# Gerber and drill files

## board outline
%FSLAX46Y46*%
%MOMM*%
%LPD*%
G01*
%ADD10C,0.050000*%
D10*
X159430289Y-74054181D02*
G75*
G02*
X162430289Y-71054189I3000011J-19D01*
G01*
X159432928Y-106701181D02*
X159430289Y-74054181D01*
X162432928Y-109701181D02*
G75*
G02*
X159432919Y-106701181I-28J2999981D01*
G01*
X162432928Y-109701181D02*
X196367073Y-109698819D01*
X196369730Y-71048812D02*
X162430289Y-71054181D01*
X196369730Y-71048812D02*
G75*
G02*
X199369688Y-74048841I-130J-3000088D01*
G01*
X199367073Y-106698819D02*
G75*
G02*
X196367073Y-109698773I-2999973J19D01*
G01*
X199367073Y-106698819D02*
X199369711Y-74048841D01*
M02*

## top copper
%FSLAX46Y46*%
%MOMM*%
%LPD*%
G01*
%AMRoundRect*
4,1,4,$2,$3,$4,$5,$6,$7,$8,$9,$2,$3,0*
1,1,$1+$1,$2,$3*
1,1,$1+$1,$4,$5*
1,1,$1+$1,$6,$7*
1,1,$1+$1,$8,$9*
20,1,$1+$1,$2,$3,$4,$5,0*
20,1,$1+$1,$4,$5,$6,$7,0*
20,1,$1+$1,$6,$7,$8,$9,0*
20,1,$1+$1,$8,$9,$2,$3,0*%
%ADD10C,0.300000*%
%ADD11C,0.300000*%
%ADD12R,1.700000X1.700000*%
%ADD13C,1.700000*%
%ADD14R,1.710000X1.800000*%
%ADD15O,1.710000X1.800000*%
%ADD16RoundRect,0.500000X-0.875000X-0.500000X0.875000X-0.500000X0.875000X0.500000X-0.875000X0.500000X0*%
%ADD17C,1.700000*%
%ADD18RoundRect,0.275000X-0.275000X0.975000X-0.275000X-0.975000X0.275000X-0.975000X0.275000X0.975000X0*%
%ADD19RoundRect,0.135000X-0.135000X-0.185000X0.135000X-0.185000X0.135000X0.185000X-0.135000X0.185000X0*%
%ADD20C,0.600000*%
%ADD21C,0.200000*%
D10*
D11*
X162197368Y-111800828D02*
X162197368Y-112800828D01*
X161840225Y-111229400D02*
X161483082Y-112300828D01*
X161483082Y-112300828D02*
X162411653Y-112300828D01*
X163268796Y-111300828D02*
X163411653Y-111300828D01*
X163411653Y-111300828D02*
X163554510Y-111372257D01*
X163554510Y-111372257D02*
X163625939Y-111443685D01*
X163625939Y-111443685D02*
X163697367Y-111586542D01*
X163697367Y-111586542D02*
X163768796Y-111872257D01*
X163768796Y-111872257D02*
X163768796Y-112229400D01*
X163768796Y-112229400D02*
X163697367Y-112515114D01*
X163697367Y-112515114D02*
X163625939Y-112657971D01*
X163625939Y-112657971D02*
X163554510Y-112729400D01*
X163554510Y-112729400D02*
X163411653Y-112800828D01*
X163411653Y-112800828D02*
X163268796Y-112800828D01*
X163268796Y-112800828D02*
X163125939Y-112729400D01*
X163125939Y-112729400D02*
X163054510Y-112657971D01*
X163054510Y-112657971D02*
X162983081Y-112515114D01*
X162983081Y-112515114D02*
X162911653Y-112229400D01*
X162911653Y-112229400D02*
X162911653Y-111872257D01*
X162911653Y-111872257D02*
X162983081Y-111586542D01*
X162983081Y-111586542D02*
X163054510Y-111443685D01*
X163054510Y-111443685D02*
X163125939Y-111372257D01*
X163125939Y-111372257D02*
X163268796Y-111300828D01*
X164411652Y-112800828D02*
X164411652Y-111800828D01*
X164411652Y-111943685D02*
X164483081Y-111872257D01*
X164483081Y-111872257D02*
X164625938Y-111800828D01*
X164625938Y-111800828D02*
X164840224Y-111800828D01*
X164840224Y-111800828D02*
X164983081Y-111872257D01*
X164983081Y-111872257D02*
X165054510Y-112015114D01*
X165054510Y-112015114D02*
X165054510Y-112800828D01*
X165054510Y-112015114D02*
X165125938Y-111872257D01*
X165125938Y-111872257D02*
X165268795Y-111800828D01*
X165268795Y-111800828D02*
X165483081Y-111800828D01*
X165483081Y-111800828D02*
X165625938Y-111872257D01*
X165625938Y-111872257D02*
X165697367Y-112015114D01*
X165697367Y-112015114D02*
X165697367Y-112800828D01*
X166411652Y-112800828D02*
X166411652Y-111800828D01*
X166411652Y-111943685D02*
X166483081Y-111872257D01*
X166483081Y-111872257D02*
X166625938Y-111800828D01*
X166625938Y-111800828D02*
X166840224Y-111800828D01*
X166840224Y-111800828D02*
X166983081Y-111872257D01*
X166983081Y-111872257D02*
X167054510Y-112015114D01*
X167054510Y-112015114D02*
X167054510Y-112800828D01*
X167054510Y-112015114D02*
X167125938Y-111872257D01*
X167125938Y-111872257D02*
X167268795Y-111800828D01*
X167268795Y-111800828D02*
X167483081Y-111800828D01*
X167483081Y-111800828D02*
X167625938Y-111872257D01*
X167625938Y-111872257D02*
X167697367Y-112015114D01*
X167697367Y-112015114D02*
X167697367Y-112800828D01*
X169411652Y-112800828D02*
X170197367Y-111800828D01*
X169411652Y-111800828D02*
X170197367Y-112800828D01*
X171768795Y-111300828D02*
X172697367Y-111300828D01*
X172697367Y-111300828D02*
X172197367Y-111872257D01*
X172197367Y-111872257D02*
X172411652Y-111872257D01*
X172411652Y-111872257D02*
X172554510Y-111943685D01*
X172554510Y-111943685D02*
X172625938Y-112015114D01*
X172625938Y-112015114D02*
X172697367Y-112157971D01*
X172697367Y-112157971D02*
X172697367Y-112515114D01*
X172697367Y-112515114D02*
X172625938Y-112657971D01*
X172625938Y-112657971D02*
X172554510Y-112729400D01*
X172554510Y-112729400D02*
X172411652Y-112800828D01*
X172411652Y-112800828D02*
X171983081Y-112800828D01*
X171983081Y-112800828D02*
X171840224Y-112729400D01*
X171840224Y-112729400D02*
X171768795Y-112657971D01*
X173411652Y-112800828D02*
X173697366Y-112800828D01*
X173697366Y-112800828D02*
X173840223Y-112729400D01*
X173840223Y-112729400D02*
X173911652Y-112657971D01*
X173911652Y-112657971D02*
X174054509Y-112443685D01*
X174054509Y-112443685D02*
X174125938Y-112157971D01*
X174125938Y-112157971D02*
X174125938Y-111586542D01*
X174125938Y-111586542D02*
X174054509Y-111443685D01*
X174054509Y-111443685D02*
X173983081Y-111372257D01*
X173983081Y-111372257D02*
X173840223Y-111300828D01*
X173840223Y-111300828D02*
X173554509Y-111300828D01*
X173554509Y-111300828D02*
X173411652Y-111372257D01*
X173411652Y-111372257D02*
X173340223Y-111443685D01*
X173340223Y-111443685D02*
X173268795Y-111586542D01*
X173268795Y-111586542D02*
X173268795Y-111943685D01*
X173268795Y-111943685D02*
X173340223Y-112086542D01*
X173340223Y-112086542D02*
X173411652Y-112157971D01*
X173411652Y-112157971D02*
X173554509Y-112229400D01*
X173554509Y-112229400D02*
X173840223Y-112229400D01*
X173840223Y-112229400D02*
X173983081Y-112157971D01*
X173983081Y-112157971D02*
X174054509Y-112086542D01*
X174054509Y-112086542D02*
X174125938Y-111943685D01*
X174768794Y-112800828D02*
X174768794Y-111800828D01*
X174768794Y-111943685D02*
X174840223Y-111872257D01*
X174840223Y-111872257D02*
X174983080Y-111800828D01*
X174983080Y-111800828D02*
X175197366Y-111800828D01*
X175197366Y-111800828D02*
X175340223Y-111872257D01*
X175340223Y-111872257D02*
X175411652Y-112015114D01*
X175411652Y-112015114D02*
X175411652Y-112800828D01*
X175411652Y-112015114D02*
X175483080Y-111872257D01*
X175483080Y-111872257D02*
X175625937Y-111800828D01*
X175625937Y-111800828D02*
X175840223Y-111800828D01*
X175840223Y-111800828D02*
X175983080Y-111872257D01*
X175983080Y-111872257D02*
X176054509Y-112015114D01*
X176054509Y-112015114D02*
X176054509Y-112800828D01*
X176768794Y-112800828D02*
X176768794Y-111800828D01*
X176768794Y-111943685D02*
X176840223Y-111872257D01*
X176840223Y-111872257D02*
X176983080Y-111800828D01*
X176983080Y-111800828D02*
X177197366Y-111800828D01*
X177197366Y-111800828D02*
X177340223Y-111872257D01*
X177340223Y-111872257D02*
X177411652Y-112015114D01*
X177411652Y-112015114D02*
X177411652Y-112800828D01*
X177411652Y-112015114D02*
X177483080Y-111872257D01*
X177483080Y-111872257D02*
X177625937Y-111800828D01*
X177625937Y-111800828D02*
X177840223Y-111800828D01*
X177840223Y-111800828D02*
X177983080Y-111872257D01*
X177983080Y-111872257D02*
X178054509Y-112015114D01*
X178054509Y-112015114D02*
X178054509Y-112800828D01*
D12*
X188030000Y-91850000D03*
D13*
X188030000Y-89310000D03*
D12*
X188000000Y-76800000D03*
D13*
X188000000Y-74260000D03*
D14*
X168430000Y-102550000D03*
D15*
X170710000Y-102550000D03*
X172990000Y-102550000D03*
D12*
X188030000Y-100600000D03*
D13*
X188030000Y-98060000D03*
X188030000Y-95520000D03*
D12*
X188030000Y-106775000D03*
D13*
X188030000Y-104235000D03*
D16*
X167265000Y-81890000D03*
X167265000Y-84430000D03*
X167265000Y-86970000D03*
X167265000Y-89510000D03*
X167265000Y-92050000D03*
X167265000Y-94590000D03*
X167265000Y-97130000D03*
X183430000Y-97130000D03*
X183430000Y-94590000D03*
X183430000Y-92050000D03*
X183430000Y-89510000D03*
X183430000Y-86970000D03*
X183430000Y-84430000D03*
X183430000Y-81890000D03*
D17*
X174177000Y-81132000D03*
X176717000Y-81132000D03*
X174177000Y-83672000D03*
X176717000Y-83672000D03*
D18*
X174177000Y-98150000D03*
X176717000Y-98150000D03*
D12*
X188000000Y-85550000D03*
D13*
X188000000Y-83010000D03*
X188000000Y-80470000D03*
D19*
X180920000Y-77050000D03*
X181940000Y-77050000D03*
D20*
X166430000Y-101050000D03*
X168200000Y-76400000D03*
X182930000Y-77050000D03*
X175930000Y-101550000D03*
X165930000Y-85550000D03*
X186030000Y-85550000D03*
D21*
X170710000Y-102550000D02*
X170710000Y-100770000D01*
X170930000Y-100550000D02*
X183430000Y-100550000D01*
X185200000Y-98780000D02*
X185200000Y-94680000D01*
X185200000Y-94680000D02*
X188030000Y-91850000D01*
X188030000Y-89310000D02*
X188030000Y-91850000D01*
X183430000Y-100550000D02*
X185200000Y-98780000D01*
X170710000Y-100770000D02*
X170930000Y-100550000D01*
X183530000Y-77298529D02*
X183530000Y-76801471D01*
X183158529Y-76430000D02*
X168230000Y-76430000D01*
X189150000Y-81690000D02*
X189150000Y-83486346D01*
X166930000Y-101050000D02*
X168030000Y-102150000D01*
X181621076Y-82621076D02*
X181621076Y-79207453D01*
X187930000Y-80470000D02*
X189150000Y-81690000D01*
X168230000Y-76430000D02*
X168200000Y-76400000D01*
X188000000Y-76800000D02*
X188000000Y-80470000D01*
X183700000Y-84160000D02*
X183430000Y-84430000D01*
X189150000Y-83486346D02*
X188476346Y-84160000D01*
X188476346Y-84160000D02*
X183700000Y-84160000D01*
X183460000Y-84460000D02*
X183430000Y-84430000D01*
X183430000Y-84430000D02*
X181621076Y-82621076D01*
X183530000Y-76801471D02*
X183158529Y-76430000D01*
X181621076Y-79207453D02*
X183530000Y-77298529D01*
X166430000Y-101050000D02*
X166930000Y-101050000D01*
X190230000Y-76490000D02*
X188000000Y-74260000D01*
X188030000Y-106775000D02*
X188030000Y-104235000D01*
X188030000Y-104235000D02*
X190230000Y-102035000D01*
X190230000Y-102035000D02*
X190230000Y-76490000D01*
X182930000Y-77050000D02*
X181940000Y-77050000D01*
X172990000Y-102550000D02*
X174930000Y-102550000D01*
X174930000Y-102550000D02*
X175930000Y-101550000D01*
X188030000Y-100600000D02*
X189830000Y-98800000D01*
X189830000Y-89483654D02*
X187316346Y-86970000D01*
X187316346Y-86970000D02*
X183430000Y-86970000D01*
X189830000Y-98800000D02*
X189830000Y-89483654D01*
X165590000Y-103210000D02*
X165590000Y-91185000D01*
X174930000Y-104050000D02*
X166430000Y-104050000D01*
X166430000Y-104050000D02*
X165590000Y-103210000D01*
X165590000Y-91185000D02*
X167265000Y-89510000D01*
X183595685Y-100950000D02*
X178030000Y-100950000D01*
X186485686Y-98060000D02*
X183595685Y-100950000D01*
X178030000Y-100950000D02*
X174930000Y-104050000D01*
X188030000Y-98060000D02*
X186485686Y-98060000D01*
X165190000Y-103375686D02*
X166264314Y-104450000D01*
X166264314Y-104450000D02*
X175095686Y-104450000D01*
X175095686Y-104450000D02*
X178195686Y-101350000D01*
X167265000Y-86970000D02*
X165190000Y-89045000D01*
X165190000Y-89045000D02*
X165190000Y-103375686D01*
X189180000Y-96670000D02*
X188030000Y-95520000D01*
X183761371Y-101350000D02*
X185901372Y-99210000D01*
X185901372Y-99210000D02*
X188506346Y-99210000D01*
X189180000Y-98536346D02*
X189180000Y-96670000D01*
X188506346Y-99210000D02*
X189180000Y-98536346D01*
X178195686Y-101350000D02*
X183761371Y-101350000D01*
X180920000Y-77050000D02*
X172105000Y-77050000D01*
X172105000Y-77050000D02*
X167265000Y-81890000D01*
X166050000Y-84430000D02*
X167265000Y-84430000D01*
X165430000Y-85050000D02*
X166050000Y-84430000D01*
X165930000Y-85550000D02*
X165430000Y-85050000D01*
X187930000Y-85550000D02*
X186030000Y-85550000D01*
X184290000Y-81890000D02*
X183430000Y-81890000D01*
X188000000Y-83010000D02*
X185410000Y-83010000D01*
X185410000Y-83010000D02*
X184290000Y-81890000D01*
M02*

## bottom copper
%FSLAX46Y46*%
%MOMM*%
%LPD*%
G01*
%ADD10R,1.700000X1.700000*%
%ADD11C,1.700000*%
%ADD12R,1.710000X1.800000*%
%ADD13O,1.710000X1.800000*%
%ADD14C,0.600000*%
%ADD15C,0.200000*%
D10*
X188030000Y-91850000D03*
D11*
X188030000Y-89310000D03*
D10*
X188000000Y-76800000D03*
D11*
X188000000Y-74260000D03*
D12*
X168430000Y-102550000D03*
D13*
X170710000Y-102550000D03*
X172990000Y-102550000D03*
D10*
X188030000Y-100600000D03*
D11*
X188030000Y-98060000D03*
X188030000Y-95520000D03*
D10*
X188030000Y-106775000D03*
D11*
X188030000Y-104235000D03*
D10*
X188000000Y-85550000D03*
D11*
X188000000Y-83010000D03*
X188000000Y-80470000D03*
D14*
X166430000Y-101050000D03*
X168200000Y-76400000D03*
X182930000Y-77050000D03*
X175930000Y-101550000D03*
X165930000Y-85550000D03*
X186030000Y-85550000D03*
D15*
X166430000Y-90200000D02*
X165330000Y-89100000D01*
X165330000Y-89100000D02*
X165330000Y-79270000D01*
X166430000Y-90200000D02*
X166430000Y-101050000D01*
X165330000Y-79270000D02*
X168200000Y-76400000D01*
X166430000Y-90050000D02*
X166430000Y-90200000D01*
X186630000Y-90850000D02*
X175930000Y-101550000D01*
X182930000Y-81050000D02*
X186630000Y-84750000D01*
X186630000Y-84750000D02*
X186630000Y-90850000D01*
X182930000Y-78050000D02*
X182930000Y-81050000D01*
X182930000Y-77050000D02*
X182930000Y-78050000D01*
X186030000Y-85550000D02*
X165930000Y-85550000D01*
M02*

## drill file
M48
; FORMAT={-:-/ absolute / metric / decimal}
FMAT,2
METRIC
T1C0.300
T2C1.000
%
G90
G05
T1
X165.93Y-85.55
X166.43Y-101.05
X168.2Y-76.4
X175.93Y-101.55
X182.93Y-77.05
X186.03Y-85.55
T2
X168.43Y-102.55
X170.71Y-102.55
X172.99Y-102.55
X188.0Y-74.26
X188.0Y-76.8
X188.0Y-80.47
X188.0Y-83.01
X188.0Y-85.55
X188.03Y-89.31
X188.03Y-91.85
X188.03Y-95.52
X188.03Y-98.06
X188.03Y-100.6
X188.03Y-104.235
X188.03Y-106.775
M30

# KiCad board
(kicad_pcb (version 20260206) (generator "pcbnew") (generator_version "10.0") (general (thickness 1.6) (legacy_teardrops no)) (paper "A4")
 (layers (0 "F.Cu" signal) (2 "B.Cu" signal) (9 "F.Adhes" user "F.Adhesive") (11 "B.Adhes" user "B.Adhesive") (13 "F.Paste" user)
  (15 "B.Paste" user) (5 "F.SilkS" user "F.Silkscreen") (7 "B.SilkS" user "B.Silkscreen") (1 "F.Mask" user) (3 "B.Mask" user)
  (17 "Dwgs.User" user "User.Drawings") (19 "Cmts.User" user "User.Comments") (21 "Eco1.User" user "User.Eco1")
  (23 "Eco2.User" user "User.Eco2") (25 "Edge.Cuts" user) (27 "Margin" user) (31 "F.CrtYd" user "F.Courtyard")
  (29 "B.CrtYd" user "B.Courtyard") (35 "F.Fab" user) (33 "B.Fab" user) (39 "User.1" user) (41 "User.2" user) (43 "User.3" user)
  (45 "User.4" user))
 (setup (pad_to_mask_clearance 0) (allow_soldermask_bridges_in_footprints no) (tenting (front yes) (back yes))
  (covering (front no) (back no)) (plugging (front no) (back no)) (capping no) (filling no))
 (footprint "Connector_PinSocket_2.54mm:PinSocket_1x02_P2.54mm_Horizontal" (layer "F.Cu") (at 188.03 91.85 180)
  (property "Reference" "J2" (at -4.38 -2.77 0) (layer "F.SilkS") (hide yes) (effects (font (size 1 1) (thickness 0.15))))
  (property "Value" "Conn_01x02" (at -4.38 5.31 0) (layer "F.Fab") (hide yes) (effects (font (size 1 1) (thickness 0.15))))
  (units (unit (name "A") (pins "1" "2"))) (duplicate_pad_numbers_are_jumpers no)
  (pad "1" thru_hole rect (at 0 0 180) (size 1.7 1.7) (drill 1) (layers "*.Cu" "*.Mask") (remove_unused_layers no) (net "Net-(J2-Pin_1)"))
  (pad "2" thru_hole circle (at 0 2.54 180) (size 1.7 1.7) (drill 1) (layers "*.Cu" "*.Mask") (remove_unused_layers no)
   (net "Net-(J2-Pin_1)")))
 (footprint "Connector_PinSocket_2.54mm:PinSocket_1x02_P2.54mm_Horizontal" (layer "F.Cu") (at 188 76.8 180)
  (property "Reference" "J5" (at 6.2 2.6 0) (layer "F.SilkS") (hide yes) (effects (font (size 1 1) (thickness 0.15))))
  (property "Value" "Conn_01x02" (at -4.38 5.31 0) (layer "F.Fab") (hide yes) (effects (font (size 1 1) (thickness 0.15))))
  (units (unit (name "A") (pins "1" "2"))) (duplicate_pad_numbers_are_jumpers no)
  (pad "1" thru_hole rect (at 0 0 180) (size 1.7 1.7) (drill 1) (layers "*.Cu" "*.Mask") (remove_unused_layers no) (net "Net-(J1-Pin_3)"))
  (pad "2" thru_hole circle (at 0 2.54 180) (size 1.7 1.7) (drill 1) (layers "*.Cu" "*.Mask") (remove_unused_layers no)
   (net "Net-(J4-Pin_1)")))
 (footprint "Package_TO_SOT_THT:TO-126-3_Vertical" (layer "F.Cu") (at 168.43 102.55)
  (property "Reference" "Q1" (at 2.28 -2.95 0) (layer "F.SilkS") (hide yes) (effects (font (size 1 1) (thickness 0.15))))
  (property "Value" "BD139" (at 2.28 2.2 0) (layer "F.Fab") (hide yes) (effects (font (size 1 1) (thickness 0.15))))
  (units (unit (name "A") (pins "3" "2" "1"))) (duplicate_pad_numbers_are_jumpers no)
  (pad "1" thru_hole rect (at 0 0) (size 1.71 1.8) (drill 1) (layers "*.Cu" "*.Mask") (remove_unused_layers no) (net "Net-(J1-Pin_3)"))
  (pad "2" thru_hole oval (at 2.28 0) (size 1.71 1.8) (drill 1) (layers "*.Cu" "*.Mask") (remove_unused_layers no) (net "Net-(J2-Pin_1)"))
  (pad "3" thru_hole oval (at 4.56 0) (size 1.71 1.8) (drill 1) (layers "*.Cu" "*.Mask") (remove_unused_layers no) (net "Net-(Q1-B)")))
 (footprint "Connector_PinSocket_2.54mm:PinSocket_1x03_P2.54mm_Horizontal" (layer "F.Cu") (at 188.03 100.6 180)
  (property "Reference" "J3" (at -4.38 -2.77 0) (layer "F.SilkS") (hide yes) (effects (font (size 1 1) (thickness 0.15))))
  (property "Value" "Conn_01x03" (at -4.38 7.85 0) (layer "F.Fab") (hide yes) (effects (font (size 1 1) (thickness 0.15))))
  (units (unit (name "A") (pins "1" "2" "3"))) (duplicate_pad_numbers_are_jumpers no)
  (pad "1" thru_hole rect (at 0 0 180) (size 1.7 1.7) (drill 1) (layers "*.Cu" "*.Mask") (remove_unused_layers no) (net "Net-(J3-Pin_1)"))
  (pad "2" thru_hole circle (at 0 2.54 180) (size 1.7 1.7) (drill 1) (layers "*.Cu" "*.Mask") (remove_unused_layers no)
   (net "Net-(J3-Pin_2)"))
  (pad "3" thru_hole circle (at 0 5.08 180) (size 1.7 1.7) (drill 1) (layers "*.Cu" "*.Mask") (remove_unused_layers no)
   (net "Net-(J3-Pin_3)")))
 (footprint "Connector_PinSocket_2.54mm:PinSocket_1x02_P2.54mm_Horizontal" (layer "F.Cu") (at 188.03 106.775 180)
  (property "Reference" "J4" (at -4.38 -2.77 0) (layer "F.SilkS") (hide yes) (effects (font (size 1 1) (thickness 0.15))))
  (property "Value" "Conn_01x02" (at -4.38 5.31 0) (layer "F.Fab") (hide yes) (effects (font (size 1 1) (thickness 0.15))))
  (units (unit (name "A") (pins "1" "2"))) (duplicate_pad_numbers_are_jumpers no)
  (pad "1" thru_hole rect (at 0 0 180) (size 1.7 1.7) (drill 1) (layers "*.Cu" "*.Mask") (remove_unused_layers no) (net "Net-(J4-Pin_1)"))
  (pad "2" thru_hole circle (at 0 2.54 180) (size 1.7 1.7) (drill 1) (layers "*.Cu" "*.Mask") (remove_unused_layers no)
   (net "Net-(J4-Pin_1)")))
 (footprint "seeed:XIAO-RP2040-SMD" (layer "F.Cu") (at 166.43 100.01)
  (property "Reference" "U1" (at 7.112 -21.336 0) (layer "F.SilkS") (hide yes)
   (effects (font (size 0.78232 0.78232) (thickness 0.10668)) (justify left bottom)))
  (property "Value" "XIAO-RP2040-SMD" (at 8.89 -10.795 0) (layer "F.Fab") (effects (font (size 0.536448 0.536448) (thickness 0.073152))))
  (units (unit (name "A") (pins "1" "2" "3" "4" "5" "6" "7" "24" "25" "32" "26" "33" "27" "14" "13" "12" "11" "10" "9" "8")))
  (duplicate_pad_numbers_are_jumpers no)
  (pad "1" smd roundrect (at 0.835 -18.12) (size 2.75 2) (layers "F.Cu" "F.Mask" "F.Paste") (roundrect_rratio 0.25)
   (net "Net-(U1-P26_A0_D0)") (solder_mask_margin 0.0508) (thermal_bridge_angle 45))
  (pad "2" smd roundrect (at 0.835 -15.58) (size 2.75 2) (layers "F.Cu" "F.Mask" "F.Paste") (roundrect_rratio 0.25) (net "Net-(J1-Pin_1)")
   (solder_mask_margin 0.0508) (thermal_bridge_angle 45))
  (pad "3" smd roundrect (at 0.835 -13.04) (size 2.75 2) (layers "F.Cu" "F.Mask" "F.Paste") (roundrect_rratio 0.25) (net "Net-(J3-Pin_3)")
   (solder_mask_margin 0.0508) (thermal_bridge_angle 45))
  (pad "4" smd roundrect (at 0.835 -10.5) (size 2.75 2) (layers "F.Cu" "F.Mask" "F.Paste") (roundrect_rratio 0.25) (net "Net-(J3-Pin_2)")
   (solder_mask_margin 0.0508) (thermal_bridge_angle 45))
  (pad "5" smd roundrect (at 0.835 -7.96) (size 2.75 2) (layers "F.Cu" "F.Mask" "F.Paste") (roundrect_rratio 0.25)
   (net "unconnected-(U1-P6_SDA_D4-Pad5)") (solder_mask_margin 0.0508) (thermal_bridge_angle 45))
  (pad "6" smd roundrect (at 0.835 -5.42) (size 2.75 2) (layers "F.Cu" "F.Mask" "F.Paste") (roundrect_rratio 0.25)
   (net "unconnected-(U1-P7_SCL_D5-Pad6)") (solder_mask_margin 0.0508) (thermal_bridge_angle 45))
  (pad "7" smd roundrect (at 0.835 -2.88) (size 2.75 2) (layers "F.Cu" "F.Mask" "F.Paste") (roundrect_rratio 0.25)
   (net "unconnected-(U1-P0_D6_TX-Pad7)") (solder_mask_margin 0.0508) (thermal_bridge_angle 45))
  (pad "8" smd roundrect (at 17 -2.88) (size 2.75 2) (layers "F.Cu" "F.Mask" "F.Paste") (roundrect_rratio 0.25)
   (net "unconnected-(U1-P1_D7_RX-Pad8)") (solder_mask_margin 0.0508) (thermal_bridge_angle 45))
  (pad "9" smd roundrect (at 17 -5.42) (size 2.75 2) (layers "F.Cu" "F.Mask" "F.Paste") (roundrect_rratio 0.25)
   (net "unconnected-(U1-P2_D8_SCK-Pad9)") (solder_mask_margin 0.0508) (thermal_bridge_angle 45))
  (pad "10" smd roundrect (at 17 -7.96) (size 2.75 2) (layers "F.Cu" "F.Mask" "F.Paste") (roundrect_rratio 0.25)
   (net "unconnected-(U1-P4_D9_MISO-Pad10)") (solder_mask_margin 0.0508) (thermal_bridge_angle 45))
  (pad "11" smd roundrect (at 17 -10.5) (size 2.75 2) (layers "F.Cu" "F.Mask" "F.Paste") (roundrect_rratio 0.25)
   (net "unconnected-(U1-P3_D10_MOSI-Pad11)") (solder_mask_margin 0.0508) (thermal_bridge_angle 45))
  (pad "12" smd roundrect (at 17 -13.04) (size 2.75 2) (layers "F.Cu" "F.Mask" "F.Paste") (roundrect_rratio 0.25) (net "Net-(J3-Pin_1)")
   (solder_mask_margin 0.0508) (thermal_bridge_angle 45))
  (pad "13" smd roundrect (at 17 -15.58) (size 2.75 2) (layers "F.Cu" "F.Mask" "F.Paste") (roundrect_rratio 0.25) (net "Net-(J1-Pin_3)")
   (solder_mask_margin 0.0508) (thermal_bridge_angle 45))
  (pad "14" smd roundrect (at 17 -18.12) (size 2.75 2) (layers "F.Cu" "F.Mask" "F.Paste") (roundrect_rratio 0.25) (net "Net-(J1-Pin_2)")
   (solder_mask_margin 0.0508) (thermal_bridge_angle 45))
  (pad "24" smd circle (at 7.747 -18.878) (size 1.7 1.7) (layers "F.Cu" "F.Mask" "F.Paste") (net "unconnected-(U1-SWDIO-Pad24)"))
  (pad "25" smd circle (at 10.287 -18.878) (size 1.7 1.7) (layers "F.Cu" "F.Mask" "F.Paste") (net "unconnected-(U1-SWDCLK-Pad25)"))
  (pad "26" smd circle (at 7.747 -16.338) (size 1.7 1.7) (layers "F.Cu" "F.Mask" "F.Paste") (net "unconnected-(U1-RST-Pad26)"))
  (pad "27" smd circle (at 10.287 -16.338) (size 1.7 1.7) (layers "F.Cu" "F.Mask" "F.Paste") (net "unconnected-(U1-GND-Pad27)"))
  (pad "32" smd roundrect (at 7.747 -1.86 270) (size 2.5 1.1) (layers "F.Cu" "F.Mask" "F.Paste") (roundrect_rratio 0.25)
   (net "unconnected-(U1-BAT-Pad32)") (thermal_bridge_angle 45))
  (pad "33" smd roundrect (at 10.287 -1.86 270) (size 2.5 1.1) (layers "F.Cu" "F.Mask" "F.Paste") (roundrect_rratio 0.25)
   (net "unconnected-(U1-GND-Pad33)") (thermal_bridge_angle 45)))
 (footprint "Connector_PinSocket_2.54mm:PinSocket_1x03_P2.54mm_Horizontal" (layer "F.Cu") (at 188 85.55 180)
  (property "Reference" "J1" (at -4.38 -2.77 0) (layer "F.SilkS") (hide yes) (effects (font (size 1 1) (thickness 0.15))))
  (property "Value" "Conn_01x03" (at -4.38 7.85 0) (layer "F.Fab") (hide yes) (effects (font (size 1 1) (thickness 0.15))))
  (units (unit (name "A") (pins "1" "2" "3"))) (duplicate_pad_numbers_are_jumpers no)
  (pad "1" thru_hole rect (at 0 0 180) (size 1.7 1.7) (drill 1) (layers "*.Cu" "*.Mask") (remove_unused_layers no) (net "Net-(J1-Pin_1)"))
  (pad "2" thru_hole circle (at 0 2.54 180) (size 1.7 1.7) (drill 1) (layers "*.Cu" "*.Mask") (remove_unused_layers no)
   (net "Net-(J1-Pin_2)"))
  (pad "3" thru_hole circle (at 0 5.08 180) (size 1.7 1.7) (drill 1) (layers "*.Cu" "*.Mask") (remove_unused_layers no)
   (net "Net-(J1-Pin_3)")))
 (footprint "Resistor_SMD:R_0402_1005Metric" (layer "F.Cu") (at 181.43 77.05)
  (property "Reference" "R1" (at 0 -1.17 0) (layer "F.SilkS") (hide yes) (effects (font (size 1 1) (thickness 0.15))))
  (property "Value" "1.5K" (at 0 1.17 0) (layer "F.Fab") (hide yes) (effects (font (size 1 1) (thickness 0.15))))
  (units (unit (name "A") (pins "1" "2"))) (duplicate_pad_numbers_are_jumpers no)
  (pad "1" smd roundrect (at -0.51 0) (size 0.54 0.64) (layers "F.Cu" "F.Mask" "F.Paste") (roundrect_rratio 0.25) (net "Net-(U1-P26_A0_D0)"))
  (pad "2" smd roundrect (at 0.51 0) (size 0.54 0.64) (layers "F.Cu" "F.Mask" "F.Paste") (roundrect_rratio 0.25) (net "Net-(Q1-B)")))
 (gr_arc (start 159.430289 74.054181) (mid 160.308969 71.932861) (end 162.430289 71.054181) (stroke (width 0.05) (type default))
  (layer "Edge.Cuts"))
 (gr_line (start 159.432928 106.701181) (end 159.430289 74.054181) (stroke (width 0.05) (type default)) (layer "Edge.Cuts"))
 (gr_arc (start 162.432928 109.701181) (mid 160.311606 108.822502) (end 159.432928 106.701181) (stroke (width 0.05) (type default))
  (layer "Edge.Cuts"))
 (gr_line (start 162.432928 109.701181) (end 196.367073 109.698819) (stroke (width 0.05) (type default)) (layer "Edge.Cuts"))
 (gr_line (start 196.36973 71.048812) (end 162.430289 71.054181) (stroke (width 0.05) (type default)) (layer "Edge.Cuts"))
 (gr_arc (start 196.36973 71.048812) (mid 198.491013 71.927543) (end 199.369711 74.048841) (stroke (width 0.05) (type default))
  (layer "Edge.Cuts"))
 (gr_arc (start 199.367073 106.698819) (mid 198.488393 108.820139) (end 196.367073 109.698819) (stroke (width 0.05) (type default))
  (layer "Edge.Cuts"))
 (gr_line (start 199.367073 106.698819) (end 199.369711 74.048841) (stroke (width 0.05) (type default)) (layer "Edge.Cuts"))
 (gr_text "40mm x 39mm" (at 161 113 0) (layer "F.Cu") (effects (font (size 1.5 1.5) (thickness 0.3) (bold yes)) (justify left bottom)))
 (segment (start 170.71 102.55) (end 170.71 100.77) (width 0.2) (layer "F.Cu") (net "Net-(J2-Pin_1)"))
 (segment (start 170.93 100.55) (end 183.43 100.55) (width 0.2) (layer "F.Cu") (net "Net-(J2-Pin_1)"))
 (segment (start 185.2 98.78) (end 185.2 94.68) (width 0.2) (layer "F.Cu") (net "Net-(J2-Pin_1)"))
 (segment (start 185.2 94.68) (end 188.03 91.85) (width 0.2) (layer "F.Cu") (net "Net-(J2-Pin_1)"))
 (segment (start 188.03 89.31) (end 188.03 91.85) (width 0.2) (layer "F.Cu") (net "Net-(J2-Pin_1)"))
 (segment (start 183.43 100.55) (end 185.2 98.78) (width 0.2) (layer "F.Cu") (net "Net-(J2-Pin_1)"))
 (segment (start 170.71 100.77) (end 170.93 100.55) (width 0.2) (layer "F.Cu") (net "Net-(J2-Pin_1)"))
 (segment (start 183.53 77.298529) (end 183.53 76.801471) (width 0.2) (layer "F.Cu") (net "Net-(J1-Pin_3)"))
 (segment (start 183.158529 76.43) (end 168.23 76.43) (width 0.2) (layer "F.Cu") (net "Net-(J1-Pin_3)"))
 (segment (start 189.15 81.69) (end 189.15 83.486346) (width 0.2) (layer "F.Cu") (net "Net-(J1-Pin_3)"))
 (segment (start 166.93 101.05) (end 168.03 102.15) (width 0.2) (layer "F.Cu") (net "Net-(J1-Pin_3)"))
 (segment (start 181.621076 82.621076) (end 181.621076 79.207453) (width 0.2) (layer "F.Cu") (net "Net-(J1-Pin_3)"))
 (segment (start 187.93 80.47) (end 189.15 81.69) (width 0.2) (layer "F.Cu") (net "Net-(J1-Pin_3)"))
 (segment (start 168.23 76.43) (end 168.2 76.4) (width 0.2) (layer "F.Cu") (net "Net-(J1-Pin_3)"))
 (segment (start 188 76.8) (end 188 80.47) (width 0.2) (layer "F.Cu") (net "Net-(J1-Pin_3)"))
 (segment (start 183.7 84.16) (end 183.43 84.43) (width 0.2) (layer "F.Cu") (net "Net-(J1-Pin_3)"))
 (segment (start 189.15 83.486346) (end 188.476346 84.16) (width 0.2) (layer "F.Cu") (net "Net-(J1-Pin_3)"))
 (segment (start 188.476346 84.16) (end 183.7 84.16) (width 0.2) (layer "F.Cu") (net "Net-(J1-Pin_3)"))
 (segment (start 183.46 84.46) (end 183.43 84.43) (width 0.2) (layer "F.Cu") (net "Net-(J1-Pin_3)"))
 (segment (start 183.43 84.43) (end 181.621076 82.621076) (width 0.2) (layer "F.Cu") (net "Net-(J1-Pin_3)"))
 (segment (start 183.53 76.801471) (end 183.158529 76.43) (width 0.2) (layer "F.Cu") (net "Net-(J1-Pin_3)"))
 (segment (start 181.621076 79.207453) (end 183.53 77.298529) (width 0.2) (layer "F.Cu") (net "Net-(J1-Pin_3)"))
 (segment (start 166.43 101.05) (end 166.93 101.05) (width 0.2) (layer "F.Cu") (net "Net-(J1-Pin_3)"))
 (via (at 166.43 101.05) (size 0.6) (drill 0.3) (layers "F.Cu" "B.Cu") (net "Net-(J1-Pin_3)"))
 (via (at 168.2 76.4) (size 0.6) (drill 0.3) (layers "F.Cu" "B.Cu") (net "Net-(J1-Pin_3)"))
 (segment (start 166.43 90.2) (end 165.33 89.1) (width 0.2) (layer "B.Cu") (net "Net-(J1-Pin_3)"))
 (segment (start 165.33 89.1) (end 165.33 79.27) (width 0.2) (layer "B.Cu") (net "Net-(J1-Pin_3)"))
 (segment (start 166.43 90.2) (end 166.43 101.05) (width 0.2) (layer "B.Cu") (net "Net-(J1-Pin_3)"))
 (segment (start 165.33 79.27) (end 168.2 76.4) (width 0.2) (layer "B.Cu") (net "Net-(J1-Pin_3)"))
 (segment (start 166.43 90.05) (end 166.43 90.2) (width 0.2) (layer "B.Cu") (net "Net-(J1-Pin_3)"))
 (segment (start 190.23 76.49) (end 188 74.26) (width 0.2) (layer "F.Cu") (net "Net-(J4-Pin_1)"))
 (segment (start 188.03 106.775) (end 188.03 104.235) (width 0.2) (layer "F.Cu") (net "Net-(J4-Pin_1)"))
 (segment (start 188.03 104.235) (end 190.23 102.035) (width 0.2) (layer "F.Cu") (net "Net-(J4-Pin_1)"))
 (segment (start 190.23 102.035) (end 190.23 76.49) (width 0.2) (layer "F.Cu") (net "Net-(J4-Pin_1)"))
 (segment (start 182.93 77.05) (end 181.94 77.05) (width 0.2) (layer "F.Cu") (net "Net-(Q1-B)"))
 (segment (start 172.99 102.55) (end 174.93 102.55) (width 0.2) (layer "F.Cu") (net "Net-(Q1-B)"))
 (segment (start 174.93 102.55) (end 175.93 101.55) (width 0.2) (layer "F.Cu") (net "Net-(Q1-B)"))
 (via (at 182.93 77.05) (size 0.6) (drill 0.3) (layers "F.Cu" "B.Cu") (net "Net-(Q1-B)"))
 (via (at 175.93 101.55) (size 0.6) (drill 0.3) (layers "F.Cu" "B.Cu") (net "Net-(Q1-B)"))
 (segment (start 186.63 90.85) (end 175.93 101.55) (width 0.2) (layer "B.Cu") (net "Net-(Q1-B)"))
 (segment (start 182.93 81.05) (end 186.63 84.75) (width 0.2) (layer "B.Cu") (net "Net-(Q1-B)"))
 (segment (start 186.63 84.75) (end 186.63 90.85) (width 0.2) (layer "B.Cu") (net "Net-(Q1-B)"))
 (segment (start 182.93 78.05) (end 182.93 81.05) (width 0.2) (layer "B.Cu") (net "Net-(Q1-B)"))
 (segment (start 182.93 77.05) (end 182.93 78.05) (width 0.2) (layer "B.Cu") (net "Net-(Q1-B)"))
 (segment (start 188.03 100.6) (end 189.83 98.8) (width 0.2) (layer "F.Cu") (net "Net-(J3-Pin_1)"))
 (segment (start 189.83 89.483654) (end 187.316346 86.97) (width 0.2) (layer "F.Cu") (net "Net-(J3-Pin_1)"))
 (segment (start 187.316346 86.97) (end 183.43 86.97) (width 0.2) (layer "F.Cu") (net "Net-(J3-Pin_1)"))
 (segment (start 189.83 98.8) (end 189.83 89.483654) (width 0.2) (layer "F.Cu") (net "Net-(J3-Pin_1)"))
 (segment (start 165.59 103.21) (end 165.59 91.185) (width 0.2) (layer "F.Cu") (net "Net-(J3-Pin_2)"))
 (segment (start 174.93 104.05) (end 166.43 104.05) (width 0.2) (layer "F.Cu") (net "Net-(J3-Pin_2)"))
 (segment (start 166.43 104.05) (end 165.59 103.21) (width 0.2) (layer "F.Cu") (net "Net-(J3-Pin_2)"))
 (segment (start 165.59 91.185) (end 167.265 89.51) (width 0.2) (layer "F.Cu") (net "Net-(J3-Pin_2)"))
 (segment (start 183.595685 100.95) (end 178.03 100.95) (width 0.2) (layer "F.Cu") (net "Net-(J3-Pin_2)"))
 (segment (start 186.485686 98.06) (end 183.595685 100.95) (width 0.2) (layer "F.Cu") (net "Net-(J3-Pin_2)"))
 (segment (start 178.03 100.95) (end 174.93 104.05) (width 0.2) (layer "F.Cu") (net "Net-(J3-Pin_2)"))
 (segment (start 188.03 98.06) (end 186.485686 98.06) (width 0.2) (layer "F.Cu") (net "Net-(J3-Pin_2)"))
 (segment (start 165.19 103.375686) (end 166.264314 104.45) (width 0.2) (layer "F.Cu") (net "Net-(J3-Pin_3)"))
 (segment (start 166.264314 104.45) (end 175.095686 104.45) (width 0.2) (layer "F.Cu") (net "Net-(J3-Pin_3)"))
 (segment (start 175.095686 104.45) (end 178.195686 101.35) (width 0.2) (layer "F.Cu") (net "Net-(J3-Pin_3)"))
 (segment (start 167.265 86.97) (end 165.19 89.045) (width 0.2) (layer "F.Cu") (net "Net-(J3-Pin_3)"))
 (segment (start 165.19 89.045) (end 165.19 103.375686) (width 0.2) (layer "F.Cu") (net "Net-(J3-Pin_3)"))
 (segment (start 189.18 96.67) (end 188.03 95.52) (width 0.2) (layer "F.Cu") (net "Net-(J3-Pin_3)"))
 (segment (start 183.761371 101.35) (end 185.901372 99.21) (width 0.2) (layer "F.Cu") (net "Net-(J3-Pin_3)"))
 (segment (start 185.901372 99.21) (end 188.506346 99.21) (width 0.2) (layer "F.Cu") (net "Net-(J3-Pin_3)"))
 (segment (start 189.18 98.536346) (end 189.18 96.67) (width 0.2) (layer "F.Cu") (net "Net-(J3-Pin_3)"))
 (segment (start 188.506346 99.21) (end 189.18 98.536346) (width 0.2) (layer "F.Cu") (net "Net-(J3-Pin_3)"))
 (segment (start 178.195686 101.35) (end 183.761371 101.35) (width 0.2) (layer "F.Cu") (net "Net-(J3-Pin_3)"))
 (segment (start 180.92 77.05) (end 172.105 77.05) (width 0.2) (layer "F.Cu") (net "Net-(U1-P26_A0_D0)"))
 (segment (start 172.105 77.05) (end 167.265 81.89) (width 0.2) (layer "F.Cu") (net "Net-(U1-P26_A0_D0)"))
 (segment (start 166.05 84.43) (end 167.265 84.43) (width 0.2) (layer "F.Cu") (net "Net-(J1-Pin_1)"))
 (segment (start 165.43 85.05) (end 166.05 84.43) (width 0.2) (layer "F.Cu") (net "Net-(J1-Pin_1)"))
 (segment (start 165.93 85.55) (end 165.43 85.05) (width 0.2) (layer "F.Cu") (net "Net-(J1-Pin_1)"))
 (segment (start 187.93 85.55) (end 186.03 85.55) (width 0.2) (layer "F.Cu") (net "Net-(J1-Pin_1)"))
 (via (at 165.93 85.55) (size 0.6) (drill 0.3) (layers "F.Cu" "B.Cu") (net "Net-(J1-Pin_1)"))
 (via (at 186.03 85.55) (size 0.6) (drill 0.3) (layers "F.Cu" "B.Cu") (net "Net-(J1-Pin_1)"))
 (segment (start 186.03 85.55) (end 165.93 85.55) (width 0.2) (layer "B.Cu") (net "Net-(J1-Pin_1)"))
 (segment (start 184.29 81.89) (end 183.43 81.89) (width 0.2) (layer "F.Cu") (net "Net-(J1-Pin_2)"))
 (segment (start 188 83.01) (end 185.41 83.01) (width 0.2) (layer "F.Cu") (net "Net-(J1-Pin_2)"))
 (segment (start 185.41 83.01) (end 184.29 81.89) (width 0.2) (layer "F.Cu") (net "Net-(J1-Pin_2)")))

